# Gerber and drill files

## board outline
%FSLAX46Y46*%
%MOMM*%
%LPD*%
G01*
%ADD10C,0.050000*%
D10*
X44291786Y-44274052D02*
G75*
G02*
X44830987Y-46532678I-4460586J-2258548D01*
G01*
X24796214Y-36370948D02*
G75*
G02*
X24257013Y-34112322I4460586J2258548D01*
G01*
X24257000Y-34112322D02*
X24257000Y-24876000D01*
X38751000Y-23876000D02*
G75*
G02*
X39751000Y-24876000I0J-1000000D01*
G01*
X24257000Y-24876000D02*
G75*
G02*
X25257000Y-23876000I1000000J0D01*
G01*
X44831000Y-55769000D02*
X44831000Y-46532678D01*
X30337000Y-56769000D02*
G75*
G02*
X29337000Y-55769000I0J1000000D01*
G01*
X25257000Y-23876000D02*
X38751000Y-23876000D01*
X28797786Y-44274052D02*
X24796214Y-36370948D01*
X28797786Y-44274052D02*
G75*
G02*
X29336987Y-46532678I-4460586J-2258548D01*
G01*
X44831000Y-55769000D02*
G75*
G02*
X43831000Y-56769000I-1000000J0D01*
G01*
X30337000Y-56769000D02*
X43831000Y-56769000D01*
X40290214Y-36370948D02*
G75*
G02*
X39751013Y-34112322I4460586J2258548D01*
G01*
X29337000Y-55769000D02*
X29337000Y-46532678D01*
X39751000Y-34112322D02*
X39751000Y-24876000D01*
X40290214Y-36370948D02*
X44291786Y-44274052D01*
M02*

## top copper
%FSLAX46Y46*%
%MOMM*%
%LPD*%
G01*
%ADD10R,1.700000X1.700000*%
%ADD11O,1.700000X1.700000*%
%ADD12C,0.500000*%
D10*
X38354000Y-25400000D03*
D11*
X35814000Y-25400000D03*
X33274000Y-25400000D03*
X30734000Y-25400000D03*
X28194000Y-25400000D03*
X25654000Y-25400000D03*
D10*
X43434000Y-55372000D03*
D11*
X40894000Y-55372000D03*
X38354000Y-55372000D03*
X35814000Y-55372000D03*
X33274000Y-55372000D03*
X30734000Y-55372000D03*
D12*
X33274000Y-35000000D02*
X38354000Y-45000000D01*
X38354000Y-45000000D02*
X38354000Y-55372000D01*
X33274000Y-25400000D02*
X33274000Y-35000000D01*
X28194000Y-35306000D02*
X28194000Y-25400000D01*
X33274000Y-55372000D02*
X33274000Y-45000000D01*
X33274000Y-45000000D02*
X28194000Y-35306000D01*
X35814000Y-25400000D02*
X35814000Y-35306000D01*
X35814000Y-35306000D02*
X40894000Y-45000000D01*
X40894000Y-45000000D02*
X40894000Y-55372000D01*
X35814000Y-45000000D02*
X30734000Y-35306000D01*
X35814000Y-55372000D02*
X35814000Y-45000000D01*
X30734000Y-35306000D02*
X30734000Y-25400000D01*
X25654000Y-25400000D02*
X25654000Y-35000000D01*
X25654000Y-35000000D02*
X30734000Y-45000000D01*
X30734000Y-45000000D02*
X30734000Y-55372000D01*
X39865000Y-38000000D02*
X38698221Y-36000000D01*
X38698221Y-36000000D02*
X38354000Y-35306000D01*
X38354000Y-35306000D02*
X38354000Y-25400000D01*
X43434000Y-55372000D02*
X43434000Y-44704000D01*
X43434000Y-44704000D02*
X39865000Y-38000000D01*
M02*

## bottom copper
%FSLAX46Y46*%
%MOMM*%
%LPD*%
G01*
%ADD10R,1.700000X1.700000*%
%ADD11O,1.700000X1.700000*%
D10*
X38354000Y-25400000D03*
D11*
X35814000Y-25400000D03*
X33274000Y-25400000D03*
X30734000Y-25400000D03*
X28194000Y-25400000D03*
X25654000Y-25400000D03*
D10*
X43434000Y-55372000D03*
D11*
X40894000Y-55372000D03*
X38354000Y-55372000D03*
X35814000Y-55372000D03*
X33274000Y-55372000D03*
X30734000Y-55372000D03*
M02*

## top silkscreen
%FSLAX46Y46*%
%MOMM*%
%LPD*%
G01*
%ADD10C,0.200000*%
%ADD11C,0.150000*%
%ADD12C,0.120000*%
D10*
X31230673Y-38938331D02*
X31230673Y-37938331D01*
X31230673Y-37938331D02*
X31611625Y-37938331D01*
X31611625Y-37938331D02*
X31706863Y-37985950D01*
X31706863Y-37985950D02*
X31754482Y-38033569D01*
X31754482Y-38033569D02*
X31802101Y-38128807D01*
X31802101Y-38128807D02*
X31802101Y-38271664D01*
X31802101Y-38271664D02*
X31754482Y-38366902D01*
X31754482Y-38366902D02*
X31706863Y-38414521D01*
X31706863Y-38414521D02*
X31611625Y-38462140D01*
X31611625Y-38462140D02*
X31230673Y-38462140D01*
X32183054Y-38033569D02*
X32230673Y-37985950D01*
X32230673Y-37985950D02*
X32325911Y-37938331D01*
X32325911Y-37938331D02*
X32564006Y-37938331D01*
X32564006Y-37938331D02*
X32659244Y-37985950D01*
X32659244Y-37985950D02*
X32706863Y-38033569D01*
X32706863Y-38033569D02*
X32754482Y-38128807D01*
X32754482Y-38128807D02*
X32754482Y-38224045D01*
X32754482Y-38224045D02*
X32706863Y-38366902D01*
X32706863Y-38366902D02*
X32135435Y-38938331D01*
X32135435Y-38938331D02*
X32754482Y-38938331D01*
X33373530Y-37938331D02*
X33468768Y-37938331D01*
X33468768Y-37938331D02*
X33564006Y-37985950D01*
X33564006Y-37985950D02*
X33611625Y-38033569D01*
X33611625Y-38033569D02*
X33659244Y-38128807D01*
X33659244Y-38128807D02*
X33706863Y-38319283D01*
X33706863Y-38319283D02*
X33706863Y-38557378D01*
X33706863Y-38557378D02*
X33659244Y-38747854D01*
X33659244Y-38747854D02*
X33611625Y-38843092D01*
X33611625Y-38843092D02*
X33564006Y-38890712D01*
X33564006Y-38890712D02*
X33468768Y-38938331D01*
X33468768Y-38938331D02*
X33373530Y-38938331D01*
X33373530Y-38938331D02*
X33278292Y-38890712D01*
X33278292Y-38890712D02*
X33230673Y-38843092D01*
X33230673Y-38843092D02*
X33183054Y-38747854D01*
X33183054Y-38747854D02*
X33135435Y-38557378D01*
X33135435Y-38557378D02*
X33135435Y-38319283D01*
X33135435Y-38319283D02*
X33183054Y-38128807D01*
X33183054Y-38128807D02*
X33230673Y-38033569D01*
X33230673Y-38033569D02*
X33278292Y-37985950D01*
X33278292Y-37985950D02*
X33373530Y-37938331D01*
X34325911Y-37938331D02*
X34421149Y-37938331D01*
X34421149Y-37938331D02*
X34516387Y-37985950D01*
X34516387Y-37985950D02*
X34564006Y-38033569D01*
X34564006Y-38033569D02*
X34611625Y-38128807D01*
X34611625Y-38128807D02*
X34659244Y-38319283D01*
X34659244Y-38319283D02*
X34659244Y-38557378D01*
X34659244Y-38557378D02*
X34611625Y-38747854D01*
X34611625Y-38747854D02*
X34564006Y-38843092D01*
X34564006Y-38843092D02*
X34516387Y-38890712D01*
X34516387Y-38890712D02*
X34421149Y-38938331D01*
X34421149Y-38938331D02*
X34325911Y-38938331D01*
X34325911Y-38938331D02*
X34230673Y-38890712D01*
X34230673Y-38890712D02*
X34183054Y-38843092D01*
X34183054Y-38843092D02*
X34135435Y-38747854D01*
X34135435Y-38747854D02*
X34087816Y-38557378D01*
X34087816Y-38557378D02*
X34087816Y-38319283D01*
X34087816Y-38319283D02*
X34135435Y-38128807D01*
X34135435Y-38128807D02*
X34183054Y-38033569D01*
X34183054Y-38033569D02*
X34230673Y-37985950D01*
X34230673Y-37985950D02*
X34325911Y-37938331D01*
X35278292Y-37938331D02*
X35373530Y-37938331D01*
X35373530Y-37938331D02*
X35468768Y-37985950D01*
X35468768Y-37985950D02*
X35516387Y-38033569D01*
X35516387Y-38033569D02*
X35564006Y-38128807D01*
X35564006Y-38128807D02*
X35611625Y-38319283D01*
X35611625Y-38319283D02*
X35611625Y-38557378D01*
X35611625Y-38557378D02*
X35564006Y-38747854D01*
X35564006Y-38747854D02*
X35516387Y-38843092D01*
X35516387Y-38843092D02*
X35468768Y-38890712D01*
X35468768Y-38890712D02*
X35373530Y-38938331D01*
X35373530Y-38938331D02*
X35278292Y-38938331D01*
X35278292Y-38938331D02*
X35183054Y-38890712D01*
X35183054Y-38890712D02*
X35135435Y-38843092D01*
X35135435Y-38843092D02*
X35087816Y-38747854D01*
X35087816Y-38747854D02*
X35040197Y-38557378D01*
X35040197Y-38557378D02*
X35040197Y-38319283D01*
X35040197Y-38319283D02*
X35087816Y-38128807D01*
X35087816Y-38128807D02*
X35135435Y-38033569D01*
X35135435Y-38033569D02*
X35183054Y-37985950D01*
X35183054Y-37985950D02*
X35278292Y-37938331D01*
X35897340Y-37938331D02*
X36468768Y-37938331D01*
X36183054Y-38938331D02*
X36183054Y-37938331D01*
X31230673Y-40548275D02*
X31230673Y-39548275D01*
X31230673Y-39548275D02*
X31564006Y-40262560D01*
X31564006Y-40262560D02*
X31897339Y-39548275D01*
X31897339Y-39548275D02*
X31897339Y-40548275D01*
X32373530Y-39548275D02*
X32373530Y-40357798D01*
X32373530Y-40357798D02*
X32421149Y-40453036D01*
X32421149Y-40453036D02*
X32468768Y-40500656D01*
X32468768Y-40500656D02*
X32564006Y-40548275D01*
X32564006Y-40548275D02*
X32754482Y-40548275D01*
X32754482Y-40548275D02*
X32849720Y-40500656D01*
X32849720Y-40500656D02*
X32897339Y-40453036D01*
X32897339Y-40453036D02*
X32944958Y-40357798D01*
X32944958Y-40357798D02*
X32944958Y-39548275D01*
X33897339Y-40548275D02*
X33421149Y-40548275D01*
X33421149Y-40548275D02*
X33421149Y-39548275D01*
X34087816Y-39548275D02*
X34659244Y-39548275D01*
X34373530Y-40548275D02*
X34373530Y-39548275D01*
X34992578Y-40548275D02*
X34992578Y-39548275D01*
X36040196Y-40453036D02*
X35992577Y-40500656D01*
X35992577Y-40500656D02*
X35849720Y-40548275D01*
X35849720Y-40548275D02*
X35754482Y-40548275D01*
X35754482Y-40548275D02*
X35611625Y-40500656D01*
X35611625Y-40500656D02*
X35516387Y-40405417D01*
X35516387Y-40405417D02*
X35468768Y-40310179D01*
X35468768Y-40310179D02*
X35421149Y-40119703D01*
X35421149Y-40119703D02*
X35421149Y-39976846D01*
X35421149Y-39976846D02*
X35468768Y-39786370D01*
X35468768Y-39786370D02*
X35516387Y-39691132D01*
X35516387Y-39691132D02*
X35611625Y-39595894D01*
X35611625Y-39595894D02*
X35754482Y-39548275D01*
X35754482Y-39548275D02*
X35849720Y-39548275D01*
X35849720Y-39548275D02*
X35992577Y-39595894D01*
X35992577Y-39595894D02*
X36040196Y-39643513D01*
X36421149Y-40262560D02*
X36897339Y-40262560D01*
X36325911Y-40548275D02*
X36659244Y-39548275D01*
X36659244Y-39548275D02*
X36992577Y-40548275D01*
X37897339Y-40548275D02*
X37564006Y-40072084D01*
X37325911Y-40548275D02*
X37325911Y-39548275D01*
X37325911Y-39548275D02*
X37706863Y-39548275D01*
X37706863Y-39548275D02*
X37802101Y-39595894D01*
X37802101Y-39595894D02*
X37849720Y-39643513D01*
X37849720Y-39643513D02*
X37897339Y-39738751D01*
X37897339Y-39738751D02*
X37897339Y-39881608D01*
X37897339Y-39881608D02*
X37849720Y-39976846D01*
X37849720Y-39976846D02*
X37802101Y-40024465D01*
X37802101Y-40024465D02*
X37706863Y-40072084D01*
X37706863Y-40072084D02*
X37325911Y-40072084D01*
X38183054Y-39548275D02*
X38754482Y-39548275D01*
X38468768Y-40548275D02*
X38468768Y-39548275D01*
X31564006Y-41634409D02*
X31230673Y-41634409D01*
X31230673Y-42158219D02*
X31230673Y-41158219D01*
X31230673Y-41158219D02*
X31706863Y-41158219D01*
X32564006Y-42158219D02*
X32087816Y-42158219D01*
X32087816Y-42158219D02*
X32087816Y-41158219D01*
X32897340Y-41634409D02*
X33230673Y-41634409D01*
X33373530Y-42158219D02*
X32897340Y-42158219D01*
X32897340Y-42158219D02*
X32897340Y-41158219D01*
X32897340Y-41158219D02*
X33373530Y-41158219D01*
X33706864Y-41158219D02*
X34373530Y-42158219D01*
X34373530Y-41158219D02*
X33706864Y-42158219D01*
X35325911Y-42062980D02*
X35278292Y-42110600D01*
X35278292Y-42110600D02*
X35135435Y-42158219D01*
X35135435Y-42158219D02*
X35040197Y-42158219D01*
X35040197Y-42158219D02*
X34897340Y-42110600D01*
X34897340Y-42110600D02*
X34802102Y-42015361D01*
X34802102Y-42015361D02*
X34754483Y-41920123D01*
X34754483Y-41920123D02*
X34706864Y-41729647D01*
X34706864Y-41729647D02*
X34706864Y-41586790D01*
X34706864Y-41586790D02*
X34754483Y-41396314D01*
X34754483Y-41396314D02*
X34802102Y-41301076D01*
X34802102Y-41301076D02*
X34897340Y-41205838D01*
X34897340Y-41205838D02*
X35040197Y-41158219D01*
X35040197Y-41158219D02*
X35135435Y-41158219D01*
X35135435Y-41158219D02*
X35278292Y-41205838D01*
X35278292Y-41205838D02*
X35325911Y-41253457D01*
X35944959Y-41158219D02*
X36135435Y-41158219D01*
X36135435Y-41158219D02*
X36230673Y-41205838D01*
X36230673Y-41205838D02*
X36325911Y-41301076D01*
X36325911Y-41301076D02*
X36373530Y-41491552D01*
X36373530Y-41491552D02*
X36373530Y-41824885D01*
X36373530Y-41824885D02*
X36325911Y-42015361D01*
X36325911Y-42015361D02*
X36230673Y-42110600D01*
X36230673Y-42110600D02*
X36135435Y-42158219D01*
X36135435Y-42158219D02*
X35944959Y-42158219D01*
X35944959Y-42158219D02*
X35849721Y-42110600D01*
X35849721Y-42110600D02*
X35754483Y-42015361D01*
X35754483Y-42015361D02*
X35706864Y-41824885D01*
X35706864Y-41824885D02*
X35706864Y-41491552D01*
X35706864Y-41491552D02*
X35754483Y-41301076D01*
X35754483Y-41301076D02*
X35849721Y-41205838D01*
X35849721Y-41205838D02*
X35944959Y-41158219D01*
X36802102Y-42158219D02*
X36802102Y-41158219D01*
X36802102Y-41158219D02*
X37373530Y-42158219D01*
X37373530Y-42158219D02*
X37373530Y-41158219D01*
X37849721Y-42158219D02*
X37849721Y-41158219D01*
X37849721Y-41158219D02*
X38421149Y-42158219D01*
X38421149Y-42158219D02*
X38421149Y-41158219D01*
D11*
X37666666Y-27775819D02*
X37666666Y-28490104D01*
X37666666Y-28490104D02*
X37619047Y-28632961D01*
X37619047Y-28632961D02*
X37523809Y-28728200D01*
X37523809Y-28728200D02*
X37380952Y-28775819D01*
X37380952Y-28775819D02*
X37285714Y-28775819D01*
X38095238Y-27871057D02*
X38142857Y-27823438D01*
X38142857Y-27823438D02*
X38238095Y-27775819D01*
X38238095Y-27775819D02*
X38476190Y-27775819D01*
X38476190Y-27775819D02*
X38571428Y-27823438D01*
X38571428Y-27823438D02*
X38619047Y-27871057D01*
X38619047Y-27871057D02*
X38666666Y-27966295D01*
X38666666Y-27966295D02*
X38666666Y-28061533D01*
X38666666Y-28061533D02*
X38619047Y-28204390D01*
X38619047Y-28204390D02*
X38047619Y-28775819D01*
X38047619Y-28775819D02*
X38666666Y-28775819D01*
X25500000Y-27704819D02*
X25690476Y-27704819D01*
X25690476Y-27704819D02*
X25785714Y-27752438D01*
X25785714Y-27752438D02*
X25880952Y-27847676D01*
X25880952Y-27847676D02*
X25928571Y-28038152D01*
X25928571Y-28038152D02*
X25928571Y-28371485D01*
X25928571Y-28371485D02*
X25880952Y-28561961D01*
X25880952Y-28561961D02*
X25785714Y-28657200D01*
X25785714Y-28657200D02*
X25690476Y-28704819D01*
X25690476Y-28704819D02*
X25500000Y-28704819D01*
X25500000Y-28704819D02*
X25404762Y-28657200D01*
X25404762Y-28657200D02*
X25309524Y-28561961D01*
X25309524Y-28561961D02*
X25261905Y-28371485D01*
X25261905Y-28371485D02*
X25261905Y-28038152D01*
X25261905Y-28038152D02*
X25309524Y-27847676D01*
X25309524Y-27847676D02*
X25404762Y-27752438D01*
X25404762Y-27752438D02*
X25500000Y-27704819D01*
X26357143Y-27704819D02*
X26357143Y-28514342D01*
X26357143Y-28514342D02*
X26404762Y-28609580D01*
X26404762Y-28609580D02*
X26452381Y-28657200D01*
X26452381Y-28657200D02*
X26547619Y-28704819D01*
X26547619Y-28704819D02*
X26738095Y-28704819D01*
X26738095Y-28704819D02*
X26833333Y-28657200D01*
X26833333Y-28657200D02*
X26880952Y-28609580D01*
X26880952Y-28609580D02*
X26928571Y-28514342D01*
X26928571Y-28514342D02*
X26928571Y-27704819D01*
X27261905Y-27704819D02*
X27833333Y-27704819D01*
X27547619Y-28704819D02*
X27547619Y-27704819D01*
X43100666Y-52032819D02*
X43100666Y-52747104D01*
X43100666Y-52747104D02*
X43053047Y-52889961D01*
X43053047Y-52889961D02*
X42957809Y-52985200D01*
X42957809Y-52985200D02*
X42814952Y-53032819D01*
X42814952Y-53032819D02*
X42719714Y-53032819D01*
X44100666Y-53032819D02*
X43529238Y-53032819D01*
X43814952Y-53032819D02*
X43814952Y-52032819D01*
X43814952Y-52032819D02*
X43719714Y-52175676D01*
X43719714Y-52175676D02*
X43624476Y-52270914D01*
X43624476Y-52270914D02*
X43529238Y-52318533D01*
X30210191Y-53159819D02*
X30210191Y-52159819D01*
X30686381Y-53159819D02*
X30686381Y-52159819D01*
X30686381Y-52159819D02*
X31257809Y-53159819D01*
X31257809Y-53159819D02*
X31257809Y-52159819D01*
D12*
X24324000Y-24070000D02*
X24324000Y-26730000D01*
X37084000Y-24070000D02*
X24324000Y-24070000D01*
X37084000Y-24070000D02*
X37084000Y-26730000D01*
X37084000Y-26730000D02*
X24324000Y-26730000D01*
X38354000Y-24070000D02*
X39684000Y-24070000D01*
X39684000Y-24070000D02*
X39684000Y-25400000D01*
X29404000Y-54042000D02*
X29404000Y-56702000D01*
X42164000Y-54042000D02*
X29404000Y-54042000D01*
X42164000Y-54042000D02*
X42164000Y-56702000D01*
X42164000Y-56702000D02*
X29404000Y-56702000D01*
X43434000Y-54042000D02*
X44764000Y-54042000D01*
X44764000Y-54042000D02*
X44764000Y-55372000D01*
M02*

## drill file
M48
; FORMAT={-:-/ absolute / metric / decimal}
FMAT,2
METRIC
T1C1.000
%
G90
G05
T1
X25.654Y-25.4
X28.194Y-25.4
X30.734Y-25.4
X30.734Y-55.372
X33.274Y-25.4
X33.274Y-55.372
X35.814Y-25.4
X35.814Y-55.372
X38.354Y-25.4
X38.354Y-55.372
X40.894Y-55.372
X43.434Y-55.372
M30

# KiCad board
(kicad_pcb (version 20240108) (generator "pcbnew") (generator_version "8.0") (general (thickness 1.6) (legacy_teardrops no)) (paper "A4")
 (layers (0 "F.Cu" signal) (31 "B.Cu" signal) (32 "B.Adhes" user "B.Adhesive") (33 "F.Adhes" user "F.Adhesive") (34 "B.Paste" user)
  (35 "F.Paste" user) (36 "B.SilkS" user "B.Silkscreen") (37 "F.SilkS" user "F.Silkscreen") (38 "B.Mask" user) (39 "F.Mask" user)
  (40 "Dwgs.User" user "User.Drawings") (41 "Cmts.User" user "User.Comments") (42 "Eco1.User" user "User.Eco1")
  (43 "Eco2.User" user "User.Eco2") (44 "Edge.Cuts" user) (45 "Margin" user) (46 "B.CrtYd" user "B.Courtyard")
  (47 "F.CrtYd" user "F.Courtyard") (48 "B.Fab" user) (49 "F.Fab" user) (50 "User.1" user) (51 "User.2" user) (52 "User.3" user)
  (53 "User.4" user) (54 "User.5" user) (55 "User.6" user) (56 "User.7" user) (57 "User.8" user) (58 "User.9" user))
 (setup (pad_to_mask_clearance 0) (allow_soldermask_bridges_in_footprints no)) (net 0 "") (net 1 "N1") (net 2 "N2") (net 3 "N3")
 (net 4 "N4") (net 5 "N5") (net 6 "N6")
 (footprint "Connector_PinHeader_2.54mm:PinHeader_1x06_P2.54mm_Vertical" (layer "F.Cu") (at 38.354 25.4 -90)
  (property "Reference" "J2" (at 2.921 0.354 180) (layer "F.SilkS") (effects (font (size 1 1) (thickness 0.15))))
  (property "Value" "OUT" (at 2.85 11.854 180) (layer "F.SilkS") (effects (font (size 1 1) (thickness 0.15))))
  (fp_line (start -1.33 14.03) (end 1.33 14.03) (stroke (width 0.12) (type solid)) (layer "F.SilkS"))
  (fp_line (start -1.33 1.27) (end -1.33 14.03) (stroke (width 0.12) (type solid)) (layer "F.SilkS"))
  (fp_line (start -1.33 1.27) (end 1.33 1.27) (stroke (width 0.12) (type solid)) (layer "F.SilkS"))
  (fp_line (start 1.33 1.27) (end 1.33 14.03) (stroke (width 0.12) (type solid)) (layer "F.SilkS"))
  (fp_line (start -1.33 0) (end -1.33 -1.33) (stroke (width 0.12) (type solid)) (layer "F.SilkS"))
  (fp_line (start -1.33 -1.33) (end 0 -1.33) (stroke (width 0.12) (type solid)) (layer "F.SilkS"))
  (pad "1" thru_hole rect (at 0 0 270) (size 1.7 1.7) (drill 1) (layers "*.Cu" "*.Mask") (remove_unused_layers no) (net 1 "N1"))
  (pad "2" thru_hole oval (at 0 2.54 270) (size 1.7 1.7) (drill 1) (layers "*.Cu" "*.Mask") (remove_unused_layers no) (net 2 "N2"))
  (pad "3" thru_hole oval (at 0 5.08 270) (size 1.7 1.7) (drill 1) (layers "*.Cu" "*.Mask") (remove_unused_layers no) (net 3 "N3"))
  (pad "4" thru_hole oval (at 0 7.62 270) (size 1.7 1.7) (drill 1) (layers "*.Cu" "*.Mask") (remove_unused_layers no) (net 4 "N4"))
  (pad "5" thru_hole oval (at 0 10.16 270) (size 1.7 1.7) (drill 1) (layers "*.Cu" "*.Mask") (remove_unused_layers no) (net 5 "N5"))
  (pad "6" thru_hole oval (at 0 12.7 270) (size 1.7 1.7) (drill 1) (layers "*.Cu" "*.Mask") (remove_unused_layers no) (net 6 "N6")))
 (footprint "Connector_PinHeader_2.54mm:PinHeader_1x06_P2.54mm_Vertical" (layer "F.Cu") (at 43.434 55.372 -90)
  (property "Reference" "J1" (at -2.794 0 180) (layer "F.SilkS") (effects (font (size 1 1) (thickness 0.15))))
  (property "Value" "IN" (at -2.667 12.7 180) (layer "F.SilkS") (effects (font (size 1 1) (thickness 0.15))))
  (fp_line (start -1.33 14.03) (end 1.33 14.03) (stroke (width 0.12) (type solid)) (layer "F.SilkS"))
  (fp_line (start -1.33 1.27) (end -1.33 14.03) (stroke (width 0.12) (type solid)) (layer "F.SilkS"))
  (fp_line (start -1.33 1.27) (end 1.33 1.27) (stroke (width 0.12) (type solid)) (layer "F.SilkS"))
  (fp_line (start 1.33 1.27) (end 1.33 14.03) (stroke (width 0.12) (type solid)) (layer "F.SilkS"))
  (fp_line (start -1.33 0) (end -1.33 -1.33) (stroke (width 0.12) (type solid)) (layer "F.SilkS"))
  (fp_line (start -1.33 -1.33) (end 0 -1.33) (stroke (width 0.12) (type solid)) (layer "F.SilkS"))
  (pad "1" thru_hole rect (at 0 0 270) (size 1.7 1.7) (drill 1) (layers "*.Cu" "*.Mask") (remove_unused_layers no) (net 1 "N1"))
  (pad "2" thru_hole oval (at 0 2.54 270) (size 1.7 1.7) (drill 1) (layers "*.Cu" "*.Mask") (remove_unused_layers no) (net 2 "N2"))
  (pad "3" thru_hole oval (at 0 5.08 270) (size 1.7 1.7) (drill 1) (layers "*.Cu" "*.Mask") (remove_unused_layers no) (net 3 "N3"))
  (pad "4" thru_hole oval (at 0 7.62 270) (size 1.7 1.7) (drill 1) (layers "*.Cu" "*.Mask") (remove_unused_layers no) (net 4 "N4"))
  (pad "5" thru_hole oval (at 0 10.16 270) (size 1.7 1.7) (drill 1) (layers "*.Cu" "*.Mask") (remove_unused_layers no) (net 5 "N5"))
  (pad "6" thru_hole oval (at 0 12.7 270) (size 1.7 1.7) (drill 1) (layers "*.Cu" "*.Mask") (remove_unused_layers no) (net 6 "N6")))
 (gr_arc (start 44.291786 44.274052) (mid 44.694334 45.371628) (end 44.831 46.532678) (stroke (width 0.05) (type default))
  (layer "Edge.Cuts"))
 (gr_arc (start 24.796214 36.370948) (mid 24.393666 35.273372) (end 24.257 34.112322) (stroke (width 0.05) (type default))
  (layer "Edge.Cuts"))
 (gr_line (start 24.257 34.112322) (end 24.257 24.876) (stroke (width 0.05) (type default)) (layer "Edge.Cuts"))
 (gr_arc (start 38.751 23.876) (mid 39.458107 24.168893) (end 39.751 24.876) (stroke (width 0.05) (type default)) (layer "Edge.Cuts"))
 (gr_arc (start 24.257 24.876) (mid 24.549893 24.168893) (end 25.257 23.876) (stroke (width 0.05) (type default)) (layer "Edge.Cuts"))
 (gr_line (start 44.831 55.769) (end 44.831 46.532678) (stroke (width 0.05) (type default)) (layer "Edge.Cuts"))
 (gr_arc (start 30.337 56.769) (mid 29.629893 56.476107) (end 29.337 55.769) (stroke (width 0.05) (type default)) (layer "Edge.Cuts"))
 (gr_line (start 25.257 23.876) (end 38.751 23.876) (stroke (width 0.05) (type default)) (layer "Edge.Cuts"))
 (gr_line (start 28.797786 44.274052) (end 24.796214 36.370948) (stroke (width 0.05) (type default)) (layer "Edge.Cuts"))
 (gr_arc (start 28.797786 44.274052) (mid 29.200334 45.371628) (end 29.337 46.532678) (stroke (width 0.05) (type default))
  (layer "Edge.Cuts"))
 (gr_arc (start 44.831 55.769) (mid 44.538107 56.476107) (end 43.831 56.769) (stroke (width 0.05) (type default)) (layer "Edge.Cuts"))
 (gr_line (start 30.337 56.769) (end 43.831 56.769) (stroke (width 0.05) (type default)) (layer "Edge.Cuts"))
 (gr_arc (start 40.290214 36.370948) (mid 39.887666 35.273372) (end 39.751 34.112322) (stroke (width 0.05) (type default))
  (layer "Edge.Cuts"))
 (gr_line (start 29.337 55.769) (end 29.337 46.532678) (stroke (width 0.05) (type default)) (layer "Edge.Cuts"))
 (gr_line (start 39.751 34.112322) (end 39.751 24.876) (stroke (width 0.05) (type default)) (layer "Edge.Cuts"))
 (gr_line (start 40.290214 36.370948) (end 44.291786 44.274052) (stroke (width 0.05) (type default)) (layer "Edge.Cuts"))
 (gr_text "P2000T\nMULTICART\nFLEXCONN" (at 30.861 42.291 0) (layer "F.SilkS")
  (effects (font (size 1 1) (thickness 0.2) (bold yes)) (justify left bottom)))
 (segment (start 33.274 35) (end 38.354 45) (width 0.5) (layer "F.Cu") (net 3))
 (segment (start 38.354 45) (end 38.354 55.372) (width 0.5) (layer "F.Cu") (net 3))
 (segment (start 33.274 25.4) (end 33.274 35) (width 0.5) (layer "F.Cu") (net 3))
 (segment (start 28.194 35.306) (end 28.194 25.4) (width 0.5) (layer "F.Cu") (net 5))
 (segment (start 33.274 55.372) (end 33.274 45) (width 0.5) (layer "F.Cu") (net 5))
 (segment (start 33.274 45) (end 28.194 35.306) (width 0.5) (layer "F.Cu") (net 5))
 (segment (start 35.814 25.4) (end 35.814 35.306) (width 0.5) (layer "F.Cu") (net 2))
 (segment (start 35.814 35.306) (end 40.894 45) (width 0.5) (layer "F.Cu") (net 2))
 (segment (start 40.894 45) (end 40.894 55.372) (width 0.5) (layer "F.Cu") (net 2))
 (segment (start 35.814 45) (end 30.734 35.306) (width 0.5) (layer "F.Cu") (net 4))
 (segment (start 35.814 55.372) (end 35.814 45) (width 0.5) (layer "F.Cu") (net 4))
 (segment (start 30.734 35.306) (end 30.734 25.4) (width 0.5) (layer "F.Cu") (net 4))
 (segment (start 25.654 25.4) (end 25.654 35) (width 0.5) (layer "F.Cu") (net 6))
 (segment (start 25.654 35) (end 30.734 45) (width 0.5) (layer "F.Cu") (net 6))
 (segment (start 30.734 45) (end 30.734 55.372) (width 0.5) (layer "F.Cu") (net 6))
 (segment (start 39.865 38) (end 38.698221 36) (width 0.5) (layer "F.Cu") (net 1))
 (segment (start 38.698221 36) (end 38.354 35.306) (width 0.5) (layer "F.Cu") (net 1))
 (segment (start 38.354 35.306) (end 38.354 25.4) (width 0.5) (layer "F.Cu") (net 1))
 (segment (start 43.434 55.372) (end 43.434 44.704) (width 0.5) (layer "F.Cu") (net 1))
 (segment (start 43.434 44.704) (end 39.865 38) (width 0.5) (layer "F.Cu") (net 1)))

